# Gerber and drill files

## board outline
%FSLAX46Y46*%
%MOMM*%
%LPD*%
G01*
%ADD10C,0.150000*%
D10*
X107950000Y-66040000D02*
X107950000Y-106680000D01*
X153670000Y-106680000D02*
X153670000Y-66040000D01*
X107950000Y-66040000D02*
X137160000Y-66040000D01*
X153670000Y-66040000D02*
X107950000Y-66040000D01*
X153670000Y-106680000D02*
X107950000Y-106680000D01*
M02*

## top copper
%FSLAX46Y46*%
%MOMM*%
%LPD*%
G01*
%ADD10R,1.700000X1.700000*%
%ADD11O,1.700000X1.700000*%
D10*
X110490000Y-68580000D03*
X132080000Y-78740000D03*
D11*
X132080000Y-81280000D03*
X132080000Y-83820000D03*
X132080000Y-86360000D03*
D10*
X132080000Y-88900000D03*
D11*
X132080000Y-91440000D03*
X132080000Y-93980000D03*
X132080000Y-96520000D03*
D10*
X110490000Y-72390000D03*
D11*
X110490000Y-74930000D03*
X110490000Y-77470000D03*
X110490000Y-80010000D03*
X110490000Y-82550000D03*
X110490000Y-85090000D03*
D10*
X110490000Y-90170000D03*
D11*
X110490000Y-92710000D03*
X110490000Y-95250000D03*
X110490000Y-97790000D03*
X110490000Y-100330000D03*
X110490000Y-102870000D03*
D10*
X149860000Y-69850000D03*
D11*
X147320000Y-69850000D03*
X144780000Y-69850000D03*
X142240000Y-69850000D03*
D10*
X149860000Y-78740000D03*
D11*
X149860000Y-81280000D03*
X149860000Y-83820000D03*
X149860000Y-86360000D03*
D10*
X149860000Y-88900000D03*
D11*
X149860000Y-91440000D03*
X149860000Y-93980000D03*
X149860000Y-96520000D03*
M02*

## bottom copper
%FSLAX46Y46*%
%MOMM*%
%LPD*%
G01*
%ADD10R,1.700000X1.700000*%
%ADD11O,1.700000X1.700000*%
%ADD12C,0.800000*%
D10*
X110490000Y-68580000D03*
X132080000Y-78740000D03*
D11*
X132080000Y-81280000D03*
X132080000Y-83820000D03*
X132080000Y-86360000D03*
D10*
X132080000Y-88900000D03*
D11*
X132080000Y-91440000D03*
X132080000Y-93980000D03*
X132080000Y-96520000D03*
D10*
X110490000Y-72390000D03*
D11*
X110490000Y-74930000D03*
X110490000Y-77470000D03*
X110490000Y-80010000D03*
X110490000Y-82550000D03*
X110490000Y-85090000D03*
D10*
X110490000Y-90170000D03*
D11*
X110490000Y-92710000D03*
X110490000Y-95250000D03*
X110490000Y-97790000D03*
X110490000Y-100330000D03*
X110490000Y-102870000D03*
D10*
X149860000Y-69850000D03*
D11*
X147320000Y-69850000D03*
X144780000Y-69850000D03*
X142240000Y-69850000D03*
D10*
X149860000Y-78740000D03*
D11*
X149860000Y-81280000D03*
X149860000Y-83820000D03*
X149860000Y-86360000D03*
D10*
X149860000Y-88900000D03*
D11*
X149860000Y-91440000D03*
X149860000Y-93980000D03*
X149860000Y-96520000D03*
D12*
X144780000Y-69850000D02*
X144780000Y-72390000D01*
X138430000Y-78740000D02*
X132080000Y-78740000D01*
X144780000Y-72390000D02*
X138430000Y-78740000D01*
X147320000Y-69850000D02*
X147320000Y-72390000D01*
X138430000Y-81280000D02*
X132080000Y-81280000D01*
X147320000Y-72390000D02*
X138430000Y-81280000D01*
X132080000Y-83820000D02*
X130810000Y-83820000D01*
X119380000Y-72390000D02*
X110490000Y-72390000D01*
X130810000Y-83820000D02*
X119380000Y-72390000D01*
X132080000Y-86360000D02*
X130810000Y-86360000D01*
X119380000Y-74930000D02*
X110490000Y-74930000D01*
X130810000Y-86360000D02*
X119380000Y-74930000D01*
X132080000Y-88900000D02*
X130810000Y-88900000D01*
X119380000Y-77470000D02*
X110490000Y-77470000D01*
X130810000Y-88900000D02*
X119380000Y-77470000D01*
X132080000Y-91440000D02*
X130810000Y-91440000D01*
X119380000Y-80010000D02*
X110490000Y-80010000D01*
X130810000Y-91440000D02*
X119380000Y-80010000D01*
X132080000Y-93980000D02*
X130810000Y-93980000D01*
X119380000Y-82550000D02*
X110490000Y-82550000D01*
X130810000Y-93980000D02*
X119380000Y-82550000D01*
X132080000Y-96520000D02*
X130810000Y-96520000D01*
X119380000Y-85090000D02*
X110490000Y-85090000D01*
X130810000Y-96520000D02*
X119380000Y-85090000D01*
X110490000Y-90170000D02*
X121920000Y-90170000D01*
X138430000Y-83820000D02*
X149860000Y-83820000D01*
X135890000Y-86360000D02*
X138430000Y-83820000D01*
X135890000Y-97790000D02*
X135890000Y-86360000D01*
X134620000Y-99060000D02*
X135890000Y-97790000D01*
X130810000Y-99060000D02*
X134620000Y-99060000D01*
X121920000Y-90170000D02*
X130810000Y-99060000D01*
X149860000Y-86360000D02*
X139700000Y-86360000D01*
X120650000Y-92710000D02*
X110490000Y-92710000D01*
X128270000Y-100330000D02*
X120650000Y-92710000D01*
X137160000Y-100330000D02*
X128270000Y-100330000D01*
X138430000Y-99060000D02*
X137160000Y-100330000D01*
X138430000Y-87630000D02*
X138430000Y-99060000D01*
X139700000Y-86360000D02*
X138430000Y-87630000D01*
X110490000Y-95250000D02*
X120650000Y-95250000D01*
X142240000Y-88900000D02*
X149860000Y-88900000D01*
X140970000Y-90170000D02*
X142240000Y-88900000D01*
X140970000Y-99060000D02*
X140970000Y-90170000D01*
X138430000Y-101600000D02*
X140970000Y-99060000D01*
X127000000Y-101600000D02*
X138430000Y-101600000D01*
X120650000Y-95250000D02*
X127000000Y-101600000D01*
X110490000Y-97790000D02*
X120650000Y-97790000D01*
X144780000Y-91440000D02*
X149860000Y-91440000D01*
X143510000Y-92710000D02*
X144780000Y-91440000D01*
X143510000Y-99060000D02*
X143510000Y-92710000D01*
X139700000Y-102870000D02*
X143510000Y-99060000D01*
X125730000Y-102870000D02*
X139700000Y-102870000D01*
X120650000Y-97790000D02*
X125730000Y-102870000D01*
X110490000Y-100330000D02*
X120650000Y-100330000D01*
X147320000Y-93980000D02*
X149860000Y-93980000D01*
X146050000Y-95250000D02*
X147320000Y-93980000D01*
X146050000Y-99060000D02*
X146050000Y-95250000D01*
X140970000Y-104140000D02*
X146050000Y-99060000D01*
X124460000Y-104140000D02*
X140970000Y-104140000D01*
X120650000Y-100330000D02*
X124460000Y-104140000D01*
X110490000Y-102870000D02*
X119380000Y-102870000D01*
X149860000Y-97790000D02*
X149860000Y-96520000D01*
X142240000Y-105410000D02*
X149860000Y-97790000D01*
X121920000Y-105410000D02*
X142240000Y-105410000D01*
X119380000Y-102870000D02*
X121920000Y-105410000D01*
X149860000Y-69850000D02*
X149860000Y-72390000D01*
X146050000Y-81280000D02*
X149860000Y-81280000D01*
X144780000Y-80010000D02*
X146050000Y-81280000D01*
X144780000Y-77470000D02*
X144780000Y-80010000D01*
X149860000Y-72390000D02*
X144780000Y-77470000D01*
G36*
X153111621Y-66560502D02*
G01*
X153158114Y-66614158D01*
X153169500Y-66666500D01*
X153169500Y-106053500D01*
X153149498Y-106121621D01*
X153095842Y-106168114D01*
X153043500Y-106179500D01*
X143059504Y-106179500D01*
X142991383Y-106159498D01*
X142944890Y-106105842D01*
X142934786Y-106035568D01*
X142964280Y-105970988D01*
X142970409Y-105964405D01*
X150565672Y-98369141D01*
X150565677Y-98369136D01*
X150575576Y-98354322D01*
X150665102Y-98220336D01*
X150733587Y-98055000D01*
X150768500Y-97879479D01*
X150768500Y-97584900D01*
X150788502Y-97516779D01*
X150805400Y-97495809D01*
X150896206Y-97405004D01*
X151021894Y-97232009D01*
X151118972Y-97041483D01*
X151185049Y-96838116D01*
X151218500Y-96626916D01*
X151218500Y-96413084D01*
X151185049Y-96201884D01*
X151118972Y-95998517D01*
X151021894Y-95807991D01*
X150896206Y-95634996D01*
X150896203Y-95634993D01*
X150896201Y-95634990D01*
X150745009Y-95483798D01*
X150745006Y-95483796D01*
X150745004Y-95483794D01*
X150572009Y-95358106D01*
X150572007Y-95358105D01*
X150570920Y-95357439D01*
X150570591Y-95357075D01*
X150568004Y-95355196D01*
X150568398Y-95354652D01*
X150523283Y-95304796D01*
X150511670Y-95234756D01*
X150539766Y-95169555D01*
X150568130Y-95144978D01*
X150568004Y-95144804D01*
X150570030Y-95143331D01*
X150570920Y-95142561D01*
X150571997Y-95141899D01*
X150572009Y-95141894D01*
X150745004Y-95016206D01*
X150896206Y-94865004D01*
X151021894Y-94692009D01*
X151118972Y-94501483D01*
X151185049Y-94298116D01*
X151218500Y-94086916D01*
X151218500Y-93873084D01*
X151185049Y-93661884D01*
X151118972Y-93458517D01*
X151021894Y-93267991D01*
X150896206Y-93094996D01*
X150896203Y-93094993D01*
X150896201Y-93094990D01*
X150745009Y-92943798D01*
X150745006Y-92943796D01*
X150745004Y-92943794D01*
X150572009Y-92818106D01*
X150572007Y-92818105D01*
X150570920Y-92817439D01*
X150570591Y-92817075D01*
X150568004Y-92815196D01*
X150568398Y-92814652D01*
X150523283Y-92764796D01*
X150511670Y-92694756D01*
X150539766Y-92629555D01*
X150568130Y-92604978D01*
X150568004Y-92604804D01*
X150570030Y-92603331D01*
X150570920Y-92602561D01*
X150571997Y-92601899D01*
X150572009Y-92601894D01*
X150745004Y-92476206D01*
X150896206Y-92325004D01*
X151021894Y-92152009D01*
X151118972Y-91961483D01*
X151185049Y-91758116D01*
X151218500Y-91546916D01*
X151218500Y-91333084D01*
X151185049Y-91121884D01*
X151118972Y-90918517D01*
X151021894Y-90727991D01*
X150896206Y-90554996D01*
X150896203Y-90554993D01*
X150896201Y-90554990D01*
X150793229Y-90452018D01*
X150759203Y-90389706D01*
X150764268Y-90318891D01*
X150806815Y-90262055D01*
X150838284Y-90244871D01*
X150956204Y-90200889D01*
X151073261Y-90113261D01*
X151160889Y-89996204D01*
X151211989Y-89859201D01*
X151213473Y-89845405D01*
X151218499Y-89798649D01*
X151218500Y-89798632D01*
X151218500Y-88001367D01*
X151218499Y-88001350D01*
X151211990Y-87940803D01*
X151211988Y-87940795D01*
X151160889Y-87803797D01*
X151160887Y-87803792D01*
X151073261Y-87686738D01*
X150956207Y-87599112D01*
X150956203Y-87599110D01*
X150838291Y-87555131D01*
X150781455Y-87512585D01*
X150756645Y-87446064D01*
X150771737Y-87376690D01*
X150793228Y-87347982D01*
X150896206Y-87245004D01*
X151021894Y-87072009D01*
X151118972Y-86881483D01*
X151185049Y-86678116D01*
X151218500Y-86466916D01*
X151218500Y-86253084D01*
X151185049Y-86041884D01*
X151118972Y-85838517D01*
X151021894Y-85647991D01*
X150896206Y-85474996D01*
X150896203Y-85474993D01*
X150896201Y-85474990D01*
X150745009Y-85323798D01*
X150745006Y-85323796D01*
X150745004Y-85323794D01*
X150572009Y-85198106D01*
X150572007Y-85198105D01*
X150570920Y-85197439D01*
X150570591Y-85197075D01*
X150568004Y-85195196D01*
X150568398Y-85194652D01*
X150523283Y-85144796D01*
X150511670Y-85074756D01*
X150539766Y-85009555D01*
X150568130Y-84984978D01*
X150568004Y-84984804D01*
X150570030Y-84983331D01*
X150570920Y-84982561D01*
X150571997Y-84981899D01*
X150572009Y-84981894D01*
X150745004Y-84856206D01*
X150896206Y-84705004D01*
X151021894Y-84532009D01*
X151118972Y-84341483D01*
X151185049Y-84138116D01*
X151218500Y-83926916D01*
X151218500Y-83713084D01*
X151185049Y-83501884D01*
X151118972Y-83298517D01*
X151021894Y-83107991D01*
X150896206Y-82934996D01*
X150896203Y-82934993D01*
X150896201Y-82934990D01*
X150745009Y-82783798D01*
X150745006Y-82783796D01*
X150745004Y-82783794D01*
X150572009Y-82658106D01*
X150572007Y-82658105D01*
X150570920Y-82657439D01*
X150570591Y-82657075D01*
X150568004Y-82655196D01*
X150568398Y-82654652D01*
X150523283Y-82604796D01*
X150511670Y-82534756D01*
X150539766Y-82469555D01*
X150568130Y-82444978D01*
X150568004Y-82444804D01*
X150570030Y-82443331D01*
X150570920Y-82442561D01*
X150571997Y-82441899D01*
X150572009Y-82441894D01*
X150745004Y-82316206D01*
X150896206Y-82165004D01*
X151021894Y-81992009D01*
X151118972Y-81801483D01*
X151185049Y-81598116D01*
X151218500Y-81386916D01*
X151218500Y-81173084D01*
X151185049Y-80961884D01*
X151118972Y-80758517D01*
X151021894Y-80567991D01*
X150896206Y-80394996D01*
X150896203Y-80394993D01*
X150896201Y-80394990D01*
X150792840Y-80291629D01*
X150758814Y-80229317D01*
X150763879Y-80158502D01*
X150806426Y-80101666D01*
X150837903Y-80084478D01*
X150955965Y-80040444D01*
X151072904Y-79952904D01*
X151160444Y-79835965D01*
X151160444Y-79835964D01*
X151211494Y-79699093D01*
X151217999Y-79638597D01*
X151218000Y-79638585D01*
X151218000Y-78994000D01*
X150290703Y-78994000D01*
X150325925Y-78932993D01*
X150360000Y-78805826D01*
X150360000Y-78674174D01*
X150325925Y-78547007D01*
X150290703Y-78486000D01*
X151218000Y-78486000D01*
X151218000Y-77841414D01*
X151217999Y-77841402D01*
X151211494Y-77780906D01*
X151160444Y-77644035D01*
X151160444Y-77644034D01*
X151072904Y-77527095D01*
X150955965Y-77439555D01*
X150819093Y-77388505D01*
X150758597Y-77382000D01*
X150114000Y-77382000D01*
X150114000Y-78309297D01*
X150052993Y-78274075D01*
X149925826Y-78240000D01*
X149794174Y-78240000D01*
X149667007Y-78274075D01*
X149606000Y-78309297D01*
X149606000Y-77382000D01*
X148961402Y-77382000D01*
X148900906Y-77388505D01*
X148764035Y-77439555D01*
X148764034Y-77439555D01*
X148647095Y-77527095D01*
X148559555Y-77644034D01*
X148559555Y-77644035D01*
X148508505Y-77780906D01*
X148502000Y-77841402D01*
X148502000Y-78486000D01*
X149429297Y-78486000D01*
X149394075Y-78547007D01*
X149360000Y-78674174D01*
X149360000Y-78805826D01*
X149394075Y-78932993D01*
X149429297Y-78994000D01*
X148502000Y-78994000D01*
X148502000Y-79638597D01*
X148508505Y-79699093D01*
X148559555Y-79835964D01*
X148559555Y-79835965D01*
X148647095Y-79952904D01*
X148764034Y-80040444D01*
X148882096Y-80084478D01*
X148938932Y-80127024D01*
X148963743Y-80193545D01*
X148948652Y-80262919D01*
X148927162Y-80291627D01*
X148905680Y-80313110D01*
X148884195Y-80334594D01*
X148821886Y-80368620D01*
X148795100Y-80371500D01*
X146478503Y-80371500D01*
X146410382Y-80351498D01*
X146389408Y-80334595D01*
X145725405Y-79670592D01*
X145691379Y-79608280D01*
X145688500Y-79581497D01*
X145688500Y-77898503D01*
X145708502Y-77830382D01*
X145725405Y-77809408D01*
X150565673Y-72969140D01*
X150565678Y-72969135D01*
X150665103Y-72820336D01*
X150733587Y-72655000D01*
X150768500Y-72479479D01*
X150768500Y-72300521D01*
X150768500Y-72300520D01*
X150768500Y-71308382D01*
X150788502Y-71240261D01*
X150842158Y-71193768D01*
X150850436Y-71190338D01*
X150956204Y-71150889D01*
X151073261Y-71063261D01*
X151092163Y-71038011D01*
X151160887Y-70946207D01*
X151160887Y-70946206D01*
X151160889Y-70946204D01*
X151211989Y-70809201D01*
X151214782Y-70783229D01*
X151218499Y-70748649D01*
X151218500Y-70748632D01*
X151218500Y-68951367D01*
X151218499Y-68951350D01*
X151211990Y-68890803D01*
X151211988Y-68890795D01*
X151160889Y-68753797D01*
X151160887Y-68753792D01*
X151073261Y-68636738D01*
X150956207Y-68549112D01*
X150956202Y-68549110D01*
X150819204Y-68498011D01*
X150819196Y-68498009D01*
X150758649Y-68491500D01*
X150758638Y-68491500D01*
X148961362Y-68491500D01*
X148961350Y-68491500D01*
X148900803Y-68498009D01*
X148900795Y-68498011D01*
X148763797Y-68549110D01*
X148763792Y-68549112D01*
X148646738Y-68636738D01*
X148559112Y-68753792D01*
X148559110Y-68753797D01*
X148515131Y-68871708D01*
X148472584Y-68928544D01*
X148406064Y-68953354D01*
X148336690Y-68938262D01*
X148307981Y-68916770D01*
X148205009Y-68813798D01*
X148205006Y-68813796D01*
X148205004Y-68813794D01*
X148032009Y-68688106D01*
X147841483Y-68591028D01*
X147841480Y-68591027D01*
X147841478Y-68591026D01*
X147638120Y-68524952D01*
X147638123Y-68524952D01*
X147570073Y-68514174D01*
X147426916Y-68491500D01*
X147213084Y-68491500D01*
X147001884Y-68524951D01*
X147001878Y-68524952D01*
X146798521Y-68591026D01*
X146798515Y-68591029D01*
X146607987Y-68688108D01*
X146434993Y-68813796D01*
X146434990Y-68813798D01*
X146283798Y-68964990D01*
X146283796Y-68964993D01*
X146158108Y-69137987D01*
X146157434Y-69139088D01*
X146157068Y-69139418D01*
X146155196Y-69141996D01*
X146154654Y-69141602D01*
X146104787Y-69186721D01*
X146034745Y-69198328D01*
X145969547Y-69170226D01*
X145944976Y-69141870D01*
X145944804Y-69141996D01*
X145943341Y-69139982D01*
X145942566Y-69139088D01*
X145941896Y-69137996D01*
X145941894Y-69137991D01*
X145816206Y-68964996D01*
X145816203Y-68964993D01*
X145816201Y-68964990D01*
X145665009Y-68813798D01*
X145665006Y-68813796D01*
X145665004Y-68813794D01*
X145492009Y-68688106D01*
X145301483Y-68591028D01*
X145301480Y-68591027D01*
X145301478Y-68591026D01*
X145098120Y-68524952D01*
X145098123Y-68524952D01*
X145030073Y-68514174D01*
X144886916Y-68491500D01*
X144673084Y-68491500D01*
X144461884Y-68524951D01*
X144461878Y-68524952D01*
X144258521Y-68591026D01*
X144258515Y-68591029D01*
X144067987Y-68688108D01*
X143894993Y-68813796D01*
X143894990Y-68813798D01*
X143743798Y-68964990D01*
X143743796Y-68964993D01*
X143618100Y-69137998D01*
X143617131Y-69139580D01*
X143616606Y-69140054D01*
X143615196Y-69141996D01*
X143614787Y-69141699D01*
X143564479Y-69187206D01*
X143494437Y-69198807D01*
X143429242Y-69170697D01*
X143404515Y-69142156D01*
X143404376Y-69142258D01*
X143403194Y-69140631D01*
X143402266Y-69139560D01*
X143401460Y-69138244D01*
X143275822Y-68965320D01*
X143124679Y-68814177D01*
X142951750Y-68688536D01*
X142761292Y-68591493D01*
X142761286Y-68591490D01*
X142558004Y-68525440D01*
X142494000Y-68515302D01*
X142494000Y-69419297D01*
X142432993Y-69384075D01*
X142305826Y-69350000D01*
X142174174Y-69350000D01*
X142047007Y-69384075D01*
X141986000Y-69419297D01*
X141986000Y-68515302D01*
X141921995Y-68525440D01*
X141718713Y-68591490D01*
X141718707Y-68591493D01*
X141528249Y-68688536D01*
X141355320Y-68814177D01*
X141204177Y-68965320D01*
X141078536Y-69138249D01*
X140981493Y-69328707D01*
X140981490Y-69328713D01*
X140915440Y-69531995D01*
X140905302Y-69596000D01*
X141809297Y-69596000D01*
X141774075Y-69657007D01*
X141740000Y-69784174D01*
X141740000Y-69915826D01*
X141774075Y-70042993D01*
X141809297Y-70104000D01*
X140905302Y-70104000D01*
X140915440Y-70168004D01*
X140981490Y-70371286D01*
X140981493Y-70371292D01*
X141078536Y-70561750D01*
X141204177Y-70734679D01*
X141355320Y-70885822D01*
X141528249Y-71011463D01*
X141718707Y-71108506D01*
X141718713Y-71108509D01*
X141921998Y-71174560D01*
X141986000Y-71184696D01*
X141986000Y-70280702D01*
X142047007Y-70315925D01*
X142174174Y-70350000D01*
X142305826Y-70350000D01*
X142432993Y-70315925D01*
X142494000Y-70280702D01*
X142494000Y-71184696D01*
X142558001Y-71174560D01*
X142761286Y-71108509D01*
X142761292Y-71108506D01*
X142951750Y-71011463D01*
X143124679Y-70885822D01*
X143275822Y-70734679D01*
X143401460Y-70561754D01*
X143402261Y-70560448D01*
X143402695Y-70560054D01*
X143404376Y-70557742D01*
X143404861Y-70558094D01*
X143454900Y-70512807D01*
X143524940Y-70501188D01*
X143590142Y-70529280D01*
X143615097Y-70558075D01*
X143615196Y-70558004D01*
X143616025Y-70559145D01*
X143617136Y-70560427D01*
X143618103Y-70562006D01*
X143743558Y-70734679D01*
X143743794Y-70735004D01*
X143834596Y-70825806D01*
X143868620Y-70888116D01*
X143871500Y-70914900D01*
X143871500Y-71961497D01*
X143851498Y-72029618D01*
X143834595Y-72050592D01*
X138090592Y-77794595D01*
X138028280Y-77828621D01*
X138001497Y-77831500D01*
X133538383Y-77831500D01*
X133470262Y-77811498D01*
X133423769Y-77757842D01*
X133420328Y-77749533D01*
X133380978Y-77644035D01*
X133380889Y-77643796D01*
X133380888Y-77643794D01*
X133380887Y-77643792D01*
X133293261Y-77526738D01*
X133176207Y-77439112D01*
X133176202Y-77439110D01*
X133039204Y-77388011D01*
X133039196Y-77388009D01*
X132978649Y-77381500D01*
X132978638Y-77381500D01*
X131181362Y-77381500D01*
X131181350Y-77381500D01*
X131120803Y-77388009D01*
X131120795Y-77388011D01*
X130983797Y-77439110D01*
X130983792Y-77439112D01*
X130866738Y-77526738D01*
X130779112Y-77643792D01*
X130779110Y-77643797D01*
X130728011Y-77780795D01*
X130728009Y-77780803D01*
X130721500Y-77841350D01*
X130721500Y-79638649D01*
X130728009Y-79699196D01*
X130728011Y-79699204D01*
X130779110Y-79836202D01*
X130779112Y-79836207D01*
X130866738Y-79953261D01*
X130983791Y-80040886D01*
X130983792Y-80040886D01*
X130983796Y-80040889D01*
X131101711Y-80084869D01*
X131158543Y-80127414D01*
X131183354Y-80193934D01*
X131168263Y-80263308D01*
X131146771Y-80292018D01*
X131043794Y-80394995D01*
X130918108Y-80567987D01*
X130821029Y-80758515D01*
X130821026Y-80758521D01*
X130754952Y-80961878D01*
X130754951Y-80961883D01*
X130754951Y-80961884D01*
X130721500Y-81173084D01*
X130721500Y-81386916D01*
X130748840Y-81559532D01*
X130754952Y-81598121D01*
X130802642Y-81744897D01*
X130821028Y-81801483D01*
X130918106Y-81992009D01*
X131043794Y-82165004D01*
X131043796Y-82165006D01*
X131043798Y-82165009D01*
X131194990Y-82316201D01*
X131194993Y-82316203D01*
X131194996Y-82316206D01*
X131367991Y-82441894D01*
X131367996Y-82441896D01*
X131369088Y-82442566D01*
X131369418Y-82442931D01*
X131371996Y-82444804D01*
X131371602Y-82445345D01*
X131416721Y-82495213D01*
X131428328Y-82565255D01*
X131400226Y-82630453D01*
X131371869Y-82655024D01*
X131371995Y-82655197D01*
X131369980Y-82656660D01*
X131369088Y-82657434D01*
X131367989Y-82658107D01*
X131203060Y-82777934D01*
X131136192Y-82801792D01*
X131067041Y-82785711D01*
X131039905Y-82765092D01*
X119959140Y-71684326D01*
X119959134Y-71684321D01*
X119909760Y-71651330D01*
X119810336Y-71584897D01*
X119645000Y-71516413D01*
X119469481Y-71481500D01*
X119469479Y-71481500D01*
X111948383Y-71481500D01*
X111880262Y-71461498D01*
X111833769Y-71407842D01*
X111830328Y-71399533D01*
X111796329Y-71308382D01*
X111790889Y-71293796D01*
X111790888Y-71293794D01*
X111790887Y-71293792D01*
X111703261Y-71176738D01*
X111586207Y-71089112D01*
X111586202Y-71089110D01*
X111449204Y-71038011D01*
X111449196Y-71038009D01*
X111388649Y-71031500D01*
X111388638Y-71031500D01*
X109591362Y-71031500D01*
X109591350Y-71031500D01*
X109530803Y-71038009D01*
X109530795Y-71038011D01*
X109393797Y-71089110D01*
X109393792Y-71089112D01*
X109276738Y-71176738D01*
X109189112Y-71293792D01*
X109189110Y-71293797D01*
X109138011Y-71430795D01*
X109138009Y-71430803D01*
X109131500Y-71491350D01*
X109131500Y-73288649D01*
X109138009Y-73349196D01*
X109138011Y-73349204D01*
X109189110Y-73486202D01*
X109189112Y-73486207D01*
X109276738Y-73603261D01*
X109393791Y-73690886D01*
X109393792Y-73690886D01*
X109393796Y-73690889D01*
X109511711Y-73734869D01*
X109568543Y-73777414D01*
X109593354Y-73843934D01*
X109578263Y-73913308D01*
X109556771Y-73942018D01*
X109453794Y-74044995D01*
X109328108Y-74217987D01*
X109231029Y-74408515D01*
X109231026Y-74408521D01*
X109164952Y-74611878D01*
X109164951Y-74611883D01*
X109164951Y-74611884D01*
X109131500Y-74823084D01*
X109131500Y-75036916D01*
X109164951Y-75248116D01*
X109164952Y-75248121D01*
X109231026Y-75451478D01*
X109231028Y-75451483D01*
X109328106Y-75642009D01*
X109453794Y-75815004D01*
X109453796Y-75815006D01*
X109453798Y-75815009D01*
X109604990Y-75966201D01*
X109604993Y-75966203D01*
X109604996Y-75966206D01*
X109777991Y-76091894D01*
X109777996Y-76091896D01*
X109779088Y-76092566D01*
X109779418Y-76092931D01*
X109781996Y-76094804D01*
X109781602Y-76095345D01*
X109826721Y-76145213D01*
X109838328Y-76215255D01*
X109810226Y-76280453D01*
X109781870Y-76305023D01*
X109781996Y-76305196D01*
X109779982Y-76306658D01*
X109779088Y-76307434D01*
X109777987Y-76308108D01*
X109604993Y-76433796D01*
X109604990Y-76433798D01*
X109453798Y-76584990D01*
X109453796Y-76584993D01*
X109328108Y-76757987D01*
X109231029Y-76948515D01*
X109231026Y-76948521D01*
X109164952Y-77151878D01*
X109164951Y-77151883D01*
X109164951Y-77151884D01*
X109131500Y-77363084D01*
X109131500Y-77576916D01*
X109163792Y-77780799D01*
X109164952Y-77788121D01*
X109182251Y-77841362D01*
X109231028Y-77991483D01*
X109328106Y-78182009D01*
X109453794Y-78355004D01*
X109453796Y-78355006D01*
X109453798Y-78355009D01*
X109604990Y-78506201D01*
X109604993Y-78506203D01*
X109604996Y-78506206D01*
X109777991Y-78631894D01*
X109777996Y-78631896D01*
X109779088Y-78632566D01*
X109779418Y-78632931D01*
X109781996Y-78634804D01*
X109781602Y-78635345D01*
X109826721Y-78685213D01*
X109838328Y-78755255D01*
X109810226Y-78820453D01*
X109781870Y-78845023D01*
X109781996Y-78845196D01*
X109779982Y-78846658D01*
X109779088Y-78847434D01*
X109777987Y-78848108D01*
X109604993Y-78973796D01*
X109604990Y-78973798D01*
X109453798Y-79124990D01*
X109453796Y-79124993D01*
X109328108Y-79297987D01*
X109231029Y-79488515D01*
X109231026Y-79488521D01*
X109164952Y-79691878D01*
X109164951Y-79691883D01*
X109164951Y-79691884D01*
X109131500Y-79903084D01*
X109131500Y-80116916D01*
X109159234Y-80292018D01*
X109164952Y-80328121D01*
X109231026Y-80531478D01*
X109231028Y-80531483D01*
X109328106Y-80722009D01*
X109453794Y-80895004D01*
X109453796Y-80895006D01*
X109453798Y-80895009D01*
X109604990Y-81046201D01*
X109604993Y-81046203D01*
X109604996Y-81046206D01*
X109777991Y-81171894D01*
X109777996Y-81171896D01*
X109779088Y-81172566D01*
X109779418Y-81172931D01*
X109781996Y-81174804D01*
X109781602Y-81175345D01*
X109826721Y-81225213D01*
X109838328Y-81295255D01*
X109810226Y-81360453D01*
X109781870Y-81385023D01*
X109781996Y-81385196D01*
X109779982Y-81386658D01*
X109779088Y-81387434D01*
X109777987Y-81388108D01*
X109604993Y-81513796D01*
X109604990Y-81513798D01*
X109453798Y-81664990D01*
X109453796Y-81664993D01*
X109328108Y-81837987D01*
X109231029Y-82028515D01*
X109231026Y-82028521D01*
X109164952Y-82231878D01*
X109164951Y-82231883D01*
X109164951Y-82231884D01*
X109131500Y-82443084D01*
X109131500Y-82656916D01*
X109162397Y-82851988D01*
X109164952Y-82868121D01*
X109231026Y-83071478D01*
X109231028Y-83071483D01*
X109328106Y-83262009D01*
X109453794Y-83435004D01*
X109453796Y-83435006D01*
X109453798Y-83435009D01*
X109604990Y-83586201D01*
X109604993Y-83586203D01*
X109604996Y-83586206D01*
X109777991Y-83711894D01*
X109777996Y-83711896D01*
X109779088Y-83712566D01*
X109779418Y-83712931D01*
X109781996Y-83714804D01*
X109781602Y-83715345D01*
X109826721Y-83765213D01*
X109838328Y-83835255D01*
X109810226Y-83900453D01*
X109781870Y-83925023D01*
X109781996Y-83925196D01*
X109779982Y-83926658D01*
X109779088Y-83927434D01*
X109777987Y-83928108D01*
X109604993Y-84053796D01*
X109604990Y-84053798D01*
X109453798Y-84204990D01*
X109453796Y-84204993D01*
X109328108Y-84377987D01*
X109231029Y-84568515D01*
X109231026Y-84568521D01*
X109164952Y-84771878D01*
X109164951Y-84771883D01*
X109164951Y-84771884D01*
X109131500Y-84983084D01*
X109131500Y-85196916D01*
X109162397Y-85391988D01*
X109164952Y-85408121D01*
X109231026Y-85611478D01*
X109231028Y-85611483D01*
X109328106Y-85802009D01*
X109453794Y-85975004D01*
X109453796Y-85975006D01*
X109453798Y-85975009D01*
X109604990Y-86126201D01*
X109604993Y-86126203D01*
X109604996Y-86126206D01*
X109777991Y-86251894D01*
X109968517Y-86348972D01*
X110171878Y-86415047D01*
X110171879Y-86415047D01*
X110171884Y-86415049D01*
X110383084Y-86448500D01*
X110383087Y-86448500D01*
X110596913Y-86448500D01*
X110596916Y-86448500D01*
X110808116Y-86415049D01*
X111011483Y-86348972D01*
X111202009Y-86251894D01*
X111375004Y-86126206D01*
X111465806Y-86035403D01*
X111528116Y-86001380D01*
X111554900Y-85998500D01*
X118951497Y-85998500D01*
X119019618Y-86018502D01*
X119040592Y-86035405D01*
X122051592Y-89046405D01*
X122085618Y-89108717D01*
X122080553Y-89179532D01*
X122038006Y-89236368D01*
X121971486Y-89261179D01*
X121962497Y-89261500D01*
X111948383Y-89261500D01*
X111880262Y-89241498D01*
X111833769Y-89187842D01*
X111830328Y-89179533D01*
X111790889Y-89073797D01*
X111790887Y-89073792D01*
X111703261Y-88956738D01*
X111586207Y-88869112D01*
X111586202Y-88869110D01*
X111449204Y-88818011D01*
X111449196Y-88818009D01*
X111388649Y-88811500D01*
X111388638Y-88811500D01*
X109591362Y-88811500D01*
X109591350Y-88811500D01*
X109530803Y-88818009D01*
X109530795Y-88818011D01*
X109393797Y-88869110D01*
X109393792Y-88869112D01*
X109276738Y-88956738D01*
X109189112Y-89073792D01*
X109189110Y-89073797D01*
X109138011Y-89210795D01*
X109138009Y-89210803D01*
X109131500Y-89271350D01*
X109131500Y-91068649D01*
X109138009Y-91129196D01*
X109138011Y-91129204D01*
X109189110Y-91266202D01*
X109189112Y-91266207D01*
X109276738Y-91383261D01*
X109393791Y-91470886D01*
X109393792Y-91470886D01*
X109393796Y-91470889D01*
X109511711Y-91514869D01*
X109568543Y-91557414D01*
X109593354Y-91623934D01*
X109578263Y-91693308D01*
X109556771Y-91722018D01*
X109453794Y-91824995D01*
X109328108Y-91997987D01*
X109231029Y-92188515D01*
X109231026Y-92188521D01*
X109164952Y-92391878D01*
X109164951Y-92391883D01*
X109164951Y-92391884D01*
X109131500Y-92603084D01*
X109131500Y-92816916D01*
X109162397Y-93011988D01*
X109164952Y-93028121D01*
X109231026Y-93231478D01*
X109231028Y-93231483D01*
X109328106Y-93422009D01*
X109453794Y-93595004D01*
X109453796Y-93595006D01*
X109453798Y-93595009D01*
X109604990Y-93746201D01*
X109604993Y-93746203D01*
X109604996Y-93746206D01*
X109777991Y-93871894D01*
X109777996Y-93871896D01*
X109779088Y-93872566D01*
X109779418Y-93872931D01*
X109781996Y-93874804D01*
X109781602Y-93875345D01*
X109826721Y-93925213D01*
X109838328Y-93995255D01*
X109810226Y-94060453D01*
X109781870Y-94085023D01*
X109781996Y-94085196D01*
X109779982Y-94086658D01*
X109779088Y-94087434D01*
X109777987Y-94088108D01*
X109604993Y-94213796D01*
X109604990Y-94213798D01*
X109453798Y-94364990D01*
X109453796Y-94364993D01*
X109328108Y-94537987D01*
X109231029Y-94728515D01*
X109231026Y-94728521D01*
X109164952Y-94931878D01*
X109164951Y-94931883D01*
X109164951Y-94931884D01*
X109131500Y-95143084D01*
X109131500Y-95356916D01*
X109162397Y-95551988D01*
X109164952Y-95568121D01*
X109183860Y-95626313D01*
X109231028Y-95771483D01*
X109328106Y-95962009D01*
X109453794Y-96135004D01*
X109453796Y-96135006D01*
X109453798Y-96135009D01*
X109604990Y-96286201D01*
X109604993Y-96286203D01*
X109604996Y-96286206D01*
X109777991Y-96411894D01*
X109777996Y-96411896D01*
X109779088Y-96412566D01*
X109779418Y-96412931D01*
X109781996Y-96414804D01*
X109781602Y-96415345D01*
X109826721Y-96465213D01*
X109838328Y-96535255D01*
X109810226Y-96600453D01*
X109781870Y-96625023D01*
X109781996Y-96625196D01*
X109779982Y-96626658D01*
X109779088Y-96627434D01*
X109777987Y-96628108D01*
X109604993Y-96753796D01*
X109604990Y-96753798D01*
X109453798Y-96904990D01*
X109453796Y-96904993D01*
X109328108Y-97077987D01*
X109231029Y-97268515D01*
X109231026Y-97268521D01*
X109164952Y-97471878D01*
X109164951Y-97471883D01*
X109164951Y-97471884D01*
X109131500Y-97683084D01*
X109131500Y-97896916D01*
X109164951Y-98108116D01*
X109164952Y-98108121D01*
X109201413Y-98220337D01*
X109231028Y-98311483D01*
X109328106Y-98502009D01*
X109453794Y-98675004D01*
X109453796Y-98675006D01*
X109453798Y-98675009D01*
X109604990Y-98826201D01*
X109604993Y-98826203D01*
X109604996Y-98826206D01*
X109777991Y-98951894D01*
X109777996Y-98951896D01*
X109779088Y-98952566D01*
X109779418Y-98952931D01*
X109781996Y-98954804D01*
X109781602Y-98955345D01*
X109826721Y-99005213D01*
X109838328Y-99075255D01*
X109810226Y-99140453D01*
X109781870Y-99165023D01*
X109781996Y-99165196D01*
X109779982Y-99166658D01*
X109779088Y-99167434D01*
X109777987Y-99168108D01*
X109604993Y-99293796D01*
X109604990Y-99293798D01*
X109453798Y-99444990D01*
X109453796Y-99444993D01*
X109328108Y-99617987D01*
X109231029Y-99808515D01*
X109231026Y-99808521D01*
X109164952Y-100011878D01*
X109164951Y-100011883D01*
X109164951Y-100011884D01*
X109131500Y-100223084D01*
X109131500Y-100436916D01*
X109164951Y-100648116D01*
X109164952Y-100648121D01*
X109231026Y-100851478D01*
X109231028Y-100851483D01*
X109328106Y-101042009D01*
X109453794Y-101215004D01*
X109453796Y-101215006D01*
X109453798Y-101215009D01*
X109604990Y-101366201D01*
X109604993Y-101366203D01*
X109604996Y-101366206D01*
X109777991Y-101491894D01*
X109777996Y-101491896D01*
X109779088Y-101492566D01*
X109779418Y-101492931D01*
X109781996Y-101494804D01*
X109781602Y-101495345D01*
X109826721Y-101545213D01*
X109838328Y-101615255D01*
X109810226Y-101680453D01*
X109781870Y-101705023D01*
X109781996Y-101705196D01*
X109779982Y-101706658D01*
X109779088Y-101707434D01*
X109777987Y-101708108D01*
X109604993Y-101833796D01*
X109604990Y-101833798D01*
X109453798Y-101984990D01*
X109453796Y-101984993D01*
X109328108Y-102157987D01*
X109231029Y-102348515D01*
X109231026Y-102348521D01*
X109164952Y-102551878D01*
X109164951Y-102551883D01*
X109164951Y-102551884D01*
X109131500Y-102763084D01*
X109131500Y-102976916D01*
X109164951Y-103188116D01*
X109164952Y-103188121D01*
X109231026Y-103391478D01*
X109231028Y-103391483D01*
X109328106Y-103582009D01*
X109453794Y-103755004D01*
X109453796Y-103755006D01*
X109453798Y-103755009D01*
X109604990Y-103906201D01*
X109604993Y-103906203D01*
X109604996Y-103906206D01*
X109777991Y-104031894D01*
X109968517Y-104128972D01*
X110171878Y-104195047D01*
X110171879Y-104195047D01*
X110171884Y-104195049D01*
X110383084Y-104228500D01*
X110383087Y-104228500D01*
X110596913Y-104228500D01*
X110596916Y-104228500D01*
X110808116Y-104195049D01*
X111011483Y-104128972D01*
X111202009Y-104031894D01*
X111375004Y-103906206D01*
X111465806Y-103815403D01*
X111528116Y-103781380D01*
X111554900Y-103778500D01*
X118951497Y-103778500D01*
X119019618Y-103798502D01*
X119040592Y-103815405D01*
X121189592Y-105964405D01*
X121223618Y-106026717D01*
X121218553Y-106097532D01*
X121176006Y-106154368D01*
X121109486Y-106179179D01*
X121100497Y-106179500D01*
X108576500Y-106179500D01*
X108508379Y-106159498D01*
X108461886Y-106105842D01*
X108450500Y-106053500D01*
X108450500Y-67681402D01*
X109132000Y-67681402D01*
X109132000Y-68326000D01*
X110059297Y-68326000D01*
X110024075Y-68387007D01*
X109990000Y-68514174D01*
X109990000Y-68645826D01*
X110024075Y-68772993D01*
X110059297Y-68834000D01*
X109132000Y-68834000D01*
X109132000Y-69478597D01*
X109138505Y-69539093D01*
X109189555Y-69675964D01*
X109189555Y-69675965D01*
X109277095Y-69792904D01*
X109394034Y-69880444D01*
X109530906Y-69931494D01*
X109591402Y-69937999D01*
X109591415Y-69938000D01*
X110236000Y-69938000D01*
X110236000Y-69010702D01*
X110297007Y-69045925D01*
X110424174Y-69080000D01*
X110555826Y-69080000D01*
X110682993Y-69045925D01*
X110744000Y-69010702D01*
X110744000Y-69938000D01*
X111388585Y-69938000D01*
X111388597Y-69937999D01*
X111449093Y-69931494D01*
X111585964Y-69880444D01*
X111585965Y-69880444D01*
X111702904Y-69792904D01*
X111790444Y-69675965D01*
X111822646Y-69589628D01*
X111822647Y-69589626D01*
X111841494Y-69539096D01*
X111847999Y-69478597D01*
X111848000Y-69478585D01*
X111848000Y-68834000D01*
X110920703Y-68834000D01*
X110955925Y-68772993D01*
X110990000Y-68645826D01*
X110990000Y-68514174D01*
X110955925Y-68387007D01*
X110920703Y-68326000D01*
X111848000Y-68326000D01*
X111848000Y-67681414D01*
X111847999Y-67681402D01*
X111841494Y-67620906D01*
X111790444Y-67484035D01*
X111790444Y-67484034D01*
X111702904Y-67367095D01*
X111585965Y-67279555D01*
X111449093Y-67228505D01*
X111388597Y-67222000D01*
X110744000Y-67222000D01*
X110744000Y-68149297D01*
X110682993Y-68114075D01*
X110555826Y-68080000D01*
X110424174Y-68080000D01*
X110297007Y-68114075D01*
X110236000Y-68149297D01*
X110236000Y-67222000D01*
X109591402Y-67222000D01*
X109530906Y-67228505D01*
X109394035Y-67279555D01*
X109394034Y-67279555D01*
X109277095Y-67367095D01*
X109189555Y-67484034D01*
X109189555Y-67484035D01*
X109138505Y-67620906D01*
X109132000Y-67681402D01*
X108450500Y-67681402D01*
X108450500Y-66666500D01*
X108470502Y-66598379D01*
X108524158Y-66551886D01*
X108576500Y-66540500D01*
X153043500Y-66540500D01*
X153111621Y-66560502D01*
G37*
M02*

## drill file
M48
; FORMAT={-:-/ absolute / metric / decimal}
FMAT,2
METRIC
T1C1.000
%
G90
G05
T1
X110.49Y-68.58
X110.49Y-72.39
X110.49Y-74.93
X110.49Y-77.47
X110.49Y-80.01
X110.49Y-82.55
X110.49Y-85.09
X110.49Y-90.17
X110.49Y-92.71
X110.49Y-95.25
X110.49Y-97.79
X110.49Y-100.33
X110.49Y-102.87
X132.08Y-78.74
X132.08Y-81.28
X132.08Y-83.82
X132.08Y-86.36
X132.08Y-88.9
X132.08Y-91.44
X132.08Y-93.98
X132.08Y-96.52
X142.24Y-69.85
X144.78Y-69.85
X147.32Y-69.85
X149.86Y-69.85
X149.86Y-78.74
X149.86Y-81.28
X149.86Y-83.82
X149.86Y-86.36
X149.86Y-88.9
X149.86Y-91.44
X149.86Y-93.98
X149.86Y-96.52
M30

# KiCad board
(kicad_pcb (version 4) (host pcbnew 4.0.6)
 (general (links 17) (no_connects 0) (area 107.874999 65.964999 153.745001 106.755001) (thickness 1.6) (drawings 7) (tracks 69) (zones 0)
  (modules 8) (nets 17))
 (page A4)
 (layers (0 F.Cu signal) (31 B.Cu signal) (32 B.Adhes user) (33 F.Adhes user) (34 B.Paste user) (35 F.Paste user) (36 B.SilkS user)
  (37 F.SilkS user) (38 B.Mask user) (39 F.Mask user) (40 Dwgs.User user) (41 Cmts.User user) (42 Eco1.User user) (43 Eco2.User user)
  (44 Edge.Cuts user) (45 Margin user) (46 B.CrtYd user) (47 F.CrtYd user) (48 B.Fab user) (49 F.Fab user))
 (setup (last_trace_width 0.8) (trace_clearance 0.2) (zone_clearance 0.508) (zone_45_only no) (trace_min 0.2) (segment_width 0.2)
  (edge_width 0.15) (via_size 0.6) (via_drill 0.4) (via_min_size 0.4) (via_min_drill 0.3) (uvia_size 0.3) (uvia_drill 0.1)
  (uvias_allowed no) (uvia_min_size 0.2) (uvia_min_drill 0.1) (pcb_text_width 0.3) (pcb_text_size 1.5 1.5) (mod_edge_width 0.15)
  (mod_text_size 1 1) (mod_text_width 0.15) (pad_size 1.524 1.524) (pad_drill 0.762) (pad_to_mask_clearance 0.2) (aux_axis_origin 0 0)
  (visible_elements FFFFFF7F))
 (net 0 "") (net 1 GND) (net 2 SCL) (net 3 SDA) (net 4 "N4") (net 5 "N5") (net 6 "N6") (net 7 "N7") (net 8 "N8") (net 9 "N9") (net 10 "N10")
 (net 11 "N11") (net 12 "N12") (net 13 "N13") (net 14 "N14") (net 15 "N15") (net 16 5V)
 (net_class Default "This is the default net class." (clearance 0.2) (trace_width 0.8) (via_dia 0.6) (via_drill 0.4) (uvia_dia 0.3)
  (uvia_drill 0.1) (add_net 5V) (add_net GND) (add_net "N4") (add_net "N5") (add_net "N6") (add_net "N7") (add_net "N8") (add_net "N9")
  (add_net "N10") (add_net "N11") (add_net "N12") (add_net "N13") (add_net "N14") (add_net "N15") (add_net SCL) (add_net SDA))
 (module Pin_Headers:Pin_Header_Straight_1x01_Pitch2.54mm (layer F.Cu) (at 110.49 68.58)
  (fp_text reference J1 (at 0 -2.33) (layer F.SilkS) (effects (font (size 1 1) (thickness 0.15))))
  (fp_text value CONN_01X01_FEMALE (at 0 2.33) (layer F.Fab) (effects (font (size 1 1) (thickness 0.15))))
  (pad 1 thru_hole rect (at 0 0) (size 1.7 1.7) (drill 1) (layers *.Cu *.Mask) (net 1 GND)))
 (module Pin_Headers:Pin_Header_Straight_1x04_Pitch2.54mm (layer F.Cu) (at 132.08 78.74)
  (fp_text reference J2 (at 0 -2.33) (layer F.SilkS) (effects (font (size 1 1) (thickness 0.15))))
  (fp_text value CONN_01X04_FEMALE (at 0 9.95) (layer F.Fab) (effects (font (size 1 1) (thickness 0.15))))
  (pad 1 thru_hole rect (at 0 0) (size 1.7 1.7) (drill 1) (layers *.Cu *.Mask) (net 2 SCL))
  (pad 2 thru_hole oval (at 0 2.54) (size 1.7 1.7) (drill 1) (layers *.Cu *.Mask) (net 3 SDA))
  (pad 3 thru_hole oval (at 0 5.08) (size 1.7 1.7) (drill 1) (layers *.Cu *.Mask) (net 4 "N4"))
  (pad 4 thru_hole oval (at 0 7.62) (size 1.7 1.7) (drill 1) (layers *.Cu *.Mask) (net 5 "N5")))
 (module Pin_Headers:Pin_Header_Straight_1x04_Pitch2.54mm (layer F.Cu) (at 132.08 88.9)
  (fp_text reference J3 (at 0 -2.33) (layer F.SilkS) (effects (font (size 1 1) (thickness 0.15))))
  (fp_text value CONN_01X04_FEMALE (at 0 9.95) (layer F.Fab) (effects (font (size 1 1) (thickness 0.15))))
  (pad 1 thru_hole rect (at 0 0) (size 1.7 1.7) (drill 1) (layers *.Cu *.Mask) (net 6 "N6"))
  (pad 2 thru_hole oval (at 0 2.54) (size 1.7 1.7) (drill 1) (layers *.Cu *.Mask) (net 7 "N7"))
  (pad 3 thru_hole oval (at 0 5.08) (size 1.7 1.7) (drill 1) (layers *.Cu *.Mask) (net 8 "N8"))
  (pad 4 thru_hole oval (at 0 7.62) (size 1.7 1.7) (drill 1) (layers *.Cu *.Mask) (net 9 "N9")))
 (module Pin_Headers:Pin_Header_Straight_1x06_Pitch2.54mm (layer F.Cu) (at 110.49 72.39)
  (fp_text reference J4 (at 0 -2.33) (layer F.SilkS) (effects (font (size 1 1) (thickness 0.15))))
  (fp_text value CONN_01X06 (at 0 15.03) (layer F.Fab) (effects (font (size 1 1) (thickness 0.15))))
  (pad 1 thru_hole rect (at 0 0) (size 1.7 1.7) (drill 1) (layers *.Cu *.Mask) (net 4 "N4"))
  (pad 2 thru_hole oval (at 0 2.54) (size 1.7 1.7) (drill 1) (layers *.Cu *.Mask) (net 5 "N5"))
  (pad 3 thru_hole oval (at 0 5.08) (size 1.7 1.7) (drill 1) (layers *.Cu *.Mask) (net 6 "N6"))
  (pad 4 thru_hole oval (at 0 7.62) (size 1.7 1.7) (drill 1) (layers *.Cu *.Mask) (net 7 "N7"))
  (pad 5 thru_hole oval (at 0 10.16) (size 1.7 1.7) (drill 1) (layers *.Cu *.Mask) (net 8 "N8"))
  (pad 6 thru_hole oval (at 0 12.7) (size 1.7 1.7) (drill 1) (layers *.Cu *.Mask) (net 9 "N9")))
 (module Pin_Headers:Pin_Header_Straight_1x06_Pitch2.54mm (layer F.Cu) (at 110.49 90.17)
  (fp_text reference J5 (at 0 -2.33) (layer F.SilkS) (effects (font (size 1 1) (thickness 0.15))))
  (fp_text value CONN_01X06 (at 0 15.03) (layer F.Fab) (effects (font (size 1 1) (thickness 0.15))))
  (pad 1 thru_hole rect (at 0 0) (size 1.7 1.7) (drill 1) (layers *.Cu *.Mask) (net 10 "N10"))
  (pad 2 thru_hole oval (at 0 2.54) (size 1.7 1.7) (drill 1) (layers *.Cu *.Mask) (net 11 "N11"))
  (pad 3 thru_hole oval (at 0 5.08) (size 1.7 1.7) (drill 1) (layers *.Cu *.Mask) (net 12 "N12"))
  (pad 4 thru_hole oval (at 0 7.62) (size 1.7 1.7) (drill 1) (layers *.Cu *.Mask) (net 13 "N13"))
  (pad 5 thru_hole oval (at 0 10.16) (size 1.7 1.7) (drill 1) (layers *.Cu *.Mask) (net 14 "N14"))
  (pad 6 thru_hole oval (at 0 12.7) (size 1.7 1.7) (drill 1) (layers *.Cu *.Mask) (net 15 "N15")))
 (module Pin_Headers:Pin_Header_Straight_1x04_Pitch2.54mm (layer F.Cu) (at 149.86 69.85 270)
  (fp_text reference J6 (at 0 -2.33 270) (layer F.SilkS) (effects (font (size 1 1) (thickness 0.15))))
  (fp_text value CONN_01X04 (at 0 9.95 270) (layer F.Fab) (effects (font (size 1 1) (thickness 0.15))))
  (pad 1 thru_hole rect (at 0 0 270) (size 1.7 1.7) (drill 1) (layers *.Cu *.Mask) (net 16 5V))
  (pad 2 thru_hole oval (at 0 2.54 270) (size 1.7 1.7) (drill 1) (layers *.Cu *.Mask) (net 3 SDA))
  (pad 3 thru_hole oval (at 0 5.08 270) (size 1.7 1.7) (drill 1) (layers *.Cu *.Mask) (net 2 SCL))
  (pad 4 thru_hole oval (at 0 7.62 270) (size 1.7 1.7) (drill 1) (layers *.Cu *.Mask) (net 1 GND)))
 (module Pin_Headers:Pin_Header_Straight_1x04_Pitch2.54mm (layer F.Cu) (at 149.86 78.74)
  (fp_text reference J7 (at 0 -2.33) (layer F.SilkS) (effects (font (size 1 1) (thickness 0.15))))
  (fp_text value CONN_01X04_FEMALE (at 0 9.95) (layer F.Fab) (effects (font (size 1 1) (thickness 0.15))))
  (pad 1 thru_hole rect (at 0 0) (size 1.7 1.7) (drill 1) (layers *.Cu *.Mask) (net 1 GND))
  (pad 2 thru_hole oval (at 0 2.54) (size 1.7 1.7) (drill 1) (layers *.Cu *.Mask) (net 16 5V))
  (pad 3 thru_hole oval (at 0 5.08) (size 1.7 1.7) (drill 1) (layers *.Cu *.Mask) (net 10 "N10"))
  (pad 4 thru_hole oval (at 0 7.62) (size 1.7 1.7) (drill 1) (layers *.Cu *.Mask) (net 11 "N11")))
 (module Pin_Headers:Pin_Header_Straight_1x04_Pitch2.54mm (layer F.Cu) (at 149.86 88.9)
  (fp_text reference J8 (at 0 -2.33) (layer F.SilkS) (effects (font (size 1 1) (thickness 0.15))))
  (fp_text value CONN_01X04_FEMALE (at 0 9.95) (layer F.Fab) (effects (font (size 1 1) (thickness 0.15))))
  (pad 1 thru_hole rect (at 0 0) (size 1.7 1.7) (drill 1) (layers *.Cu *.Mask) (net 12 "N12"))
  (pad 2 thru_hole oval (at 0 2.54) (size 1.7 1.7) (drill 1) (layers *.Cu *.Mask) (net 13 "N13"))
  (pad 3 thru_hole oval (at 0 5.08) (size 1.7 1.7) (drill 1) (layers *.Cu *.Mask) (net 14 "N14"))
  (pad 4 thru_hole oval (at 0 7.62) (size 1.7 1.7) (drill 1) (layers *.Cu *.Mask) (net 15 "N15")))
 (gr_line (start 107.95 66.04) (end 107.95 106.68) (angle 90) (layer Edge.Cuts) (width 0.15))
 (gr_line (start 153.67 106.68) (end 153.67 66.04) (angle 90) (layer Edge.Cuts) (width 0.15))
 (gr_line (start 107.95 66.04) (end 137.16 66.04) (angle 90) (layer Edge.Cuts) (width 0.15))
 (gr_line (start 153.67 66.04) (end 107.95 66.04) (angle 90) (layer Edge.Cuts) (width 0.15))
 (gr_line (start 153.67 106.68) (end 107.95 106.68) (angle 90) (layer Edge.Cuts) (width 0.15))
 (segment (start 144.78 69.85) (end 144.78 72.39) (width 0.8) (layer B.Cu) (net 2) (status 400000))
 (segment (start 138.43 78.74) (end 132.08 78.74) (width 0.8) (layer B.Cu) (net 2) (status 800000))
 (segment (start 144.78 72.39) (end 138.43 78.74) (width 0.8) (layer B.Cu) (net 2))
 (segment (start 147.32 69.85) (end 147.32 72.39) (width 0.8) (layer B.Cu) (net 3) (status 400000))
 (segment (start 138.43 81.28) (end 132.08 81.28) (width 0.8) (layer B.Cu) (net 3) (status 800000))
 (segment (start 147.32 72.39) (end 138.43 81.28) (width 0.8) (layer B.Cu) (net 3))
 (segment (start 132.08 83.82) (end 130.81 83.82) (width 0.8) (layer B.Cu) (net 4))
 (segment (start 119.38 72.39) (end 110.49 72.39) (width 0.8) (layer B.Cu) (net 4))
 (segment (start 130.81 83.82) (end 119.38 72.39) (width 0.8) (layer B.Cu) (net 4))
 (segment (start 132.08 86.36) (end 130.81 86.36) (width 0.8) (layer B.Cu) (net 5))
 (segment (start 119.38 74.93) (end 110.49 74.93) (width 0.8) (layer B.Cu) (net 5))
 (segment (start 130.81 86.36) (end 119.38 74.93) (width 0.8) (layer B.Cu) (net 5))
 (segment (start 132.08 88.9) (end 130.81 88.9) (width 0.8) (layer B.Cu) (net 6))
 (segment (start 119.38 77.47) (end 110.49 77.47) (width 0.8) (layer B.Cu) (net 6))
 (segment (start 130.81 88.9) (end 119.38 77.47) (width 0.8) (layer B.Cu) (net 6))
 (segment (start 132.08 91.44) (end 130.81 91.44) (width 0.8) (layer B.Cu) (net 7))
 (segment (start 119.38 80.01) (end 110.49 80.01) (width 0.8) (layer B.Cu) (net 7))
 (segment (start 130.81 91.44) (end 119.38 80.01) (width 0.8) (layer B.Cu) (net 7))
 (segment (start 132.08 93.98) (end 130.81 93.98) (width 0.8) (layer B.Cu) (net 8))
 (segment (start 119.38 82.55) (end 110.49 82.55) (width 0.8) (layer B.Cu) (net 8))
 (segment (start 130.81 93.98) (end 119.38 82.55) (width 0.8) (layer B.Cu) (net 8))
 (segment (start 132.08 96.52) (end 130.81 96.52) (width 0.8) (layer B.Cu) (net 9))
 (segment (start 119.38 85.09) (end 110.49 85.09) (width 0.8) (layer B.Cu) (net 9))
 (segment (start 130.81 96.52) (end 119.38 85.09) (width 0.8) (layer B.Cu) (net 9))
 (segment (start 110.49 90.17) (end 121.92 90.17) (width 0.8) (layer B.Cu) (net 10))
 (segment (start 138.43 83.82) (end 149.86 83.82) (width 0.8) (layer B.Cu) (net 10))
 (segment (start 135.89 86.36) (end 138.43 83.82) (width 0.8) (layer B.Cu) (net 10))
 (segment (start 135.89 97.79) (end 135.89 86.36) (width 0.8) (layer B.Cu) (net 10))
 (segment (start 134.62 99.06) (end 135.89 97.79) (width 0.8) (layer B.Cu) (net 10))
 (segment (start 130.81 99.06) (end 134.62 99.06) (width 0.8) (layer B.Cu) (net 10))
 (segment (start 121.92 90.17) (end 130.81 99.06) (width 0.8) (layer B.Cu) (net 10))
 (segment (start 149.86 86.36) (end 139.7 86.36) (width 0.8) (layer B.Cu) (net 11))
 (segment (start 120.65 92.71) (end 110.49 92.71) (width 0.8) (layer B.Cu) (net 11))
 (segment (start 128.27 100.33) (end 120.65 92.71) (width 0.8) (layer B.Cu) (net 11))
 (segment (start 137.16 100.33) (end 128.27 100.33) (width 0.8) (layer B.Cu) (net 11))
 (segment (start 138.43 99.06) (end 137.16 100.33) (width 0.8) (layer B.Cu) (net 11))
 (segment (start 138.43 87.63) (end 138.43 99.06) (width 0.8) (layer B.Cu) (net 11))
 (segment (start 139.7 86.36) (end 138.43 87.63) (width 0.8) (layer B.Cu) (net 11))
 (segment (start 110.49 95.25) (end 120.65 95.25) (width 0.8) (layer B.Cu) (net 12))
 (segment (start 142.24 88.9) (end 149.86 88.9) (width 0.8) (layer B.Cu) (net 12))
 (segment (start 140.97 90.17) (end 142.24 88.9) (width 0.8) (layer B.Cu) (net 12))
 (segment (start 140.97 99.06) (end 140.97 90.17) (width 0.8) (layer B.Cu) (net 12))
 (segment (start 138.43 101.6) (end 140.97 99.06) (width 0.8) (layer B.Cu) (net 12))
 (segment (start 127 101.6) (end 138.43 101.6) (width 0.8) (layer B.Cu) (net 12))
 (segment (start 120.65 95.25) (end 127 101.6) (width 0.8) (layer B.Cu) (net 12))
 (segment (start 110.49 97.79) (end 120.65 97.79) (width 0.8) (layer B.Cu) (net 13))
 (segment (start 144.78 91.44) (end 149.86 91.44) (width 0.8) (layer B.Cu) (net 13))
 (segment (start 143.51 92.71) (end 144.78 91.44) (width 0.8) (layer B.Cu) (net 13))
 (segment (start 143.51 99.06) (end 143.51 92.71) (width 0.8) (layer B.Cu) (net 13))
 (segment (start 139.7 102.87) (end 143.51 99.06) (width 0.8) (layer B.Cu) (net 13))
 (segment (start 125.73 102.87) (end 139.7 102.87) (width 0.8) (layer B.Cu) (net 13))
 (segment (start 120.65 97.79) (end 125.73 102.87) (width 0.8) (layer B.Cu) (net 13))
 (segment (start 110.49 100.33) (end 120.65 100.33) (width 0.8) (layer B.Cu) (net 14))
 (segment (start 147.32 93.98) (end 149.86 93.98) (width 0.8) (layer B.Cu) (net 14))
 (segment (start 146.05 95.25) (end 147.32 93.98) (width 0.8) (layer B.Cu) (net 14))
 (segment (start 146.05 99.06) (end 146.05 95.25) (width 0.8) (layer B.Cu) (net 14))
 (segment (start 140.97 104.14) (end 146.05 99.06) (width 0.8) (layer B.Cu) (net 14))
 (segment (start 124.46 104.14) (end 140.97 104.14) (width 0.8) (layer B.Cu) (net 14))
 (segment (start 120.65 100.33) (end 124.46 104.14) (width 0.8) (layer B.Cu) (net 14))
 (segment (start 110.49 102.87) (end 119.38 102.87) (width 0.8) (layer B.Cu) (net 15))
 (segment (start 149.86 97.79) (end 149.86 96.52) (width 0.8) (layer B.Cu) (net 15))
 (segment (start 142.24 105.41) (end 149.86 97.79) (width 0.8) (layer B.Cu) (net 15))
 (segment (start 121.92 105.41) (end 142.24 105.41) (width 0.8) (layer B.Cu) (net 15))
 (segment (start 119.38 102.87) (end 121.92 105.41) (width 0.8) (layer B.Cu) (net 15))
 (segment (start 149.86 69.85) (end 149.86 72.39) (width 0.8) (layer B.Cu) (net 16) (status 400000))
 (segment (start 146.05 81.28) (end 149.86 81.28) (width 0.8) (layer B.Cu) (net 16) (status 800000))
 (segment (start 144.78 80.01) (end 146.05 81.28) (width 0.8) (layer B.Cu) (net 16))
 (segment (start 144.78 77.47) (end 144.78 80.01) (width 0.8) (layer B.Cu) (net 16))
 (segment (start 149.86 72.39) (end 144.78 77.47) (width 0.8) (layer B.Cu) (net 16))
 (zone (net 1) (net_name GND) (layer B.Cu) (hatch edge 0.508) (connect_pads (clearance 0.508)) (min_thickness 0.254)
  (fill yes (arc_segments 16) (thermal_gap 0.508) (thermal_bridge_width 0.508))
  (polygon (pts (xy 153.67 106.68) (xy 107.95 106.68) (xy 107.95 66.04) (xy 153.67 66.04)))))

